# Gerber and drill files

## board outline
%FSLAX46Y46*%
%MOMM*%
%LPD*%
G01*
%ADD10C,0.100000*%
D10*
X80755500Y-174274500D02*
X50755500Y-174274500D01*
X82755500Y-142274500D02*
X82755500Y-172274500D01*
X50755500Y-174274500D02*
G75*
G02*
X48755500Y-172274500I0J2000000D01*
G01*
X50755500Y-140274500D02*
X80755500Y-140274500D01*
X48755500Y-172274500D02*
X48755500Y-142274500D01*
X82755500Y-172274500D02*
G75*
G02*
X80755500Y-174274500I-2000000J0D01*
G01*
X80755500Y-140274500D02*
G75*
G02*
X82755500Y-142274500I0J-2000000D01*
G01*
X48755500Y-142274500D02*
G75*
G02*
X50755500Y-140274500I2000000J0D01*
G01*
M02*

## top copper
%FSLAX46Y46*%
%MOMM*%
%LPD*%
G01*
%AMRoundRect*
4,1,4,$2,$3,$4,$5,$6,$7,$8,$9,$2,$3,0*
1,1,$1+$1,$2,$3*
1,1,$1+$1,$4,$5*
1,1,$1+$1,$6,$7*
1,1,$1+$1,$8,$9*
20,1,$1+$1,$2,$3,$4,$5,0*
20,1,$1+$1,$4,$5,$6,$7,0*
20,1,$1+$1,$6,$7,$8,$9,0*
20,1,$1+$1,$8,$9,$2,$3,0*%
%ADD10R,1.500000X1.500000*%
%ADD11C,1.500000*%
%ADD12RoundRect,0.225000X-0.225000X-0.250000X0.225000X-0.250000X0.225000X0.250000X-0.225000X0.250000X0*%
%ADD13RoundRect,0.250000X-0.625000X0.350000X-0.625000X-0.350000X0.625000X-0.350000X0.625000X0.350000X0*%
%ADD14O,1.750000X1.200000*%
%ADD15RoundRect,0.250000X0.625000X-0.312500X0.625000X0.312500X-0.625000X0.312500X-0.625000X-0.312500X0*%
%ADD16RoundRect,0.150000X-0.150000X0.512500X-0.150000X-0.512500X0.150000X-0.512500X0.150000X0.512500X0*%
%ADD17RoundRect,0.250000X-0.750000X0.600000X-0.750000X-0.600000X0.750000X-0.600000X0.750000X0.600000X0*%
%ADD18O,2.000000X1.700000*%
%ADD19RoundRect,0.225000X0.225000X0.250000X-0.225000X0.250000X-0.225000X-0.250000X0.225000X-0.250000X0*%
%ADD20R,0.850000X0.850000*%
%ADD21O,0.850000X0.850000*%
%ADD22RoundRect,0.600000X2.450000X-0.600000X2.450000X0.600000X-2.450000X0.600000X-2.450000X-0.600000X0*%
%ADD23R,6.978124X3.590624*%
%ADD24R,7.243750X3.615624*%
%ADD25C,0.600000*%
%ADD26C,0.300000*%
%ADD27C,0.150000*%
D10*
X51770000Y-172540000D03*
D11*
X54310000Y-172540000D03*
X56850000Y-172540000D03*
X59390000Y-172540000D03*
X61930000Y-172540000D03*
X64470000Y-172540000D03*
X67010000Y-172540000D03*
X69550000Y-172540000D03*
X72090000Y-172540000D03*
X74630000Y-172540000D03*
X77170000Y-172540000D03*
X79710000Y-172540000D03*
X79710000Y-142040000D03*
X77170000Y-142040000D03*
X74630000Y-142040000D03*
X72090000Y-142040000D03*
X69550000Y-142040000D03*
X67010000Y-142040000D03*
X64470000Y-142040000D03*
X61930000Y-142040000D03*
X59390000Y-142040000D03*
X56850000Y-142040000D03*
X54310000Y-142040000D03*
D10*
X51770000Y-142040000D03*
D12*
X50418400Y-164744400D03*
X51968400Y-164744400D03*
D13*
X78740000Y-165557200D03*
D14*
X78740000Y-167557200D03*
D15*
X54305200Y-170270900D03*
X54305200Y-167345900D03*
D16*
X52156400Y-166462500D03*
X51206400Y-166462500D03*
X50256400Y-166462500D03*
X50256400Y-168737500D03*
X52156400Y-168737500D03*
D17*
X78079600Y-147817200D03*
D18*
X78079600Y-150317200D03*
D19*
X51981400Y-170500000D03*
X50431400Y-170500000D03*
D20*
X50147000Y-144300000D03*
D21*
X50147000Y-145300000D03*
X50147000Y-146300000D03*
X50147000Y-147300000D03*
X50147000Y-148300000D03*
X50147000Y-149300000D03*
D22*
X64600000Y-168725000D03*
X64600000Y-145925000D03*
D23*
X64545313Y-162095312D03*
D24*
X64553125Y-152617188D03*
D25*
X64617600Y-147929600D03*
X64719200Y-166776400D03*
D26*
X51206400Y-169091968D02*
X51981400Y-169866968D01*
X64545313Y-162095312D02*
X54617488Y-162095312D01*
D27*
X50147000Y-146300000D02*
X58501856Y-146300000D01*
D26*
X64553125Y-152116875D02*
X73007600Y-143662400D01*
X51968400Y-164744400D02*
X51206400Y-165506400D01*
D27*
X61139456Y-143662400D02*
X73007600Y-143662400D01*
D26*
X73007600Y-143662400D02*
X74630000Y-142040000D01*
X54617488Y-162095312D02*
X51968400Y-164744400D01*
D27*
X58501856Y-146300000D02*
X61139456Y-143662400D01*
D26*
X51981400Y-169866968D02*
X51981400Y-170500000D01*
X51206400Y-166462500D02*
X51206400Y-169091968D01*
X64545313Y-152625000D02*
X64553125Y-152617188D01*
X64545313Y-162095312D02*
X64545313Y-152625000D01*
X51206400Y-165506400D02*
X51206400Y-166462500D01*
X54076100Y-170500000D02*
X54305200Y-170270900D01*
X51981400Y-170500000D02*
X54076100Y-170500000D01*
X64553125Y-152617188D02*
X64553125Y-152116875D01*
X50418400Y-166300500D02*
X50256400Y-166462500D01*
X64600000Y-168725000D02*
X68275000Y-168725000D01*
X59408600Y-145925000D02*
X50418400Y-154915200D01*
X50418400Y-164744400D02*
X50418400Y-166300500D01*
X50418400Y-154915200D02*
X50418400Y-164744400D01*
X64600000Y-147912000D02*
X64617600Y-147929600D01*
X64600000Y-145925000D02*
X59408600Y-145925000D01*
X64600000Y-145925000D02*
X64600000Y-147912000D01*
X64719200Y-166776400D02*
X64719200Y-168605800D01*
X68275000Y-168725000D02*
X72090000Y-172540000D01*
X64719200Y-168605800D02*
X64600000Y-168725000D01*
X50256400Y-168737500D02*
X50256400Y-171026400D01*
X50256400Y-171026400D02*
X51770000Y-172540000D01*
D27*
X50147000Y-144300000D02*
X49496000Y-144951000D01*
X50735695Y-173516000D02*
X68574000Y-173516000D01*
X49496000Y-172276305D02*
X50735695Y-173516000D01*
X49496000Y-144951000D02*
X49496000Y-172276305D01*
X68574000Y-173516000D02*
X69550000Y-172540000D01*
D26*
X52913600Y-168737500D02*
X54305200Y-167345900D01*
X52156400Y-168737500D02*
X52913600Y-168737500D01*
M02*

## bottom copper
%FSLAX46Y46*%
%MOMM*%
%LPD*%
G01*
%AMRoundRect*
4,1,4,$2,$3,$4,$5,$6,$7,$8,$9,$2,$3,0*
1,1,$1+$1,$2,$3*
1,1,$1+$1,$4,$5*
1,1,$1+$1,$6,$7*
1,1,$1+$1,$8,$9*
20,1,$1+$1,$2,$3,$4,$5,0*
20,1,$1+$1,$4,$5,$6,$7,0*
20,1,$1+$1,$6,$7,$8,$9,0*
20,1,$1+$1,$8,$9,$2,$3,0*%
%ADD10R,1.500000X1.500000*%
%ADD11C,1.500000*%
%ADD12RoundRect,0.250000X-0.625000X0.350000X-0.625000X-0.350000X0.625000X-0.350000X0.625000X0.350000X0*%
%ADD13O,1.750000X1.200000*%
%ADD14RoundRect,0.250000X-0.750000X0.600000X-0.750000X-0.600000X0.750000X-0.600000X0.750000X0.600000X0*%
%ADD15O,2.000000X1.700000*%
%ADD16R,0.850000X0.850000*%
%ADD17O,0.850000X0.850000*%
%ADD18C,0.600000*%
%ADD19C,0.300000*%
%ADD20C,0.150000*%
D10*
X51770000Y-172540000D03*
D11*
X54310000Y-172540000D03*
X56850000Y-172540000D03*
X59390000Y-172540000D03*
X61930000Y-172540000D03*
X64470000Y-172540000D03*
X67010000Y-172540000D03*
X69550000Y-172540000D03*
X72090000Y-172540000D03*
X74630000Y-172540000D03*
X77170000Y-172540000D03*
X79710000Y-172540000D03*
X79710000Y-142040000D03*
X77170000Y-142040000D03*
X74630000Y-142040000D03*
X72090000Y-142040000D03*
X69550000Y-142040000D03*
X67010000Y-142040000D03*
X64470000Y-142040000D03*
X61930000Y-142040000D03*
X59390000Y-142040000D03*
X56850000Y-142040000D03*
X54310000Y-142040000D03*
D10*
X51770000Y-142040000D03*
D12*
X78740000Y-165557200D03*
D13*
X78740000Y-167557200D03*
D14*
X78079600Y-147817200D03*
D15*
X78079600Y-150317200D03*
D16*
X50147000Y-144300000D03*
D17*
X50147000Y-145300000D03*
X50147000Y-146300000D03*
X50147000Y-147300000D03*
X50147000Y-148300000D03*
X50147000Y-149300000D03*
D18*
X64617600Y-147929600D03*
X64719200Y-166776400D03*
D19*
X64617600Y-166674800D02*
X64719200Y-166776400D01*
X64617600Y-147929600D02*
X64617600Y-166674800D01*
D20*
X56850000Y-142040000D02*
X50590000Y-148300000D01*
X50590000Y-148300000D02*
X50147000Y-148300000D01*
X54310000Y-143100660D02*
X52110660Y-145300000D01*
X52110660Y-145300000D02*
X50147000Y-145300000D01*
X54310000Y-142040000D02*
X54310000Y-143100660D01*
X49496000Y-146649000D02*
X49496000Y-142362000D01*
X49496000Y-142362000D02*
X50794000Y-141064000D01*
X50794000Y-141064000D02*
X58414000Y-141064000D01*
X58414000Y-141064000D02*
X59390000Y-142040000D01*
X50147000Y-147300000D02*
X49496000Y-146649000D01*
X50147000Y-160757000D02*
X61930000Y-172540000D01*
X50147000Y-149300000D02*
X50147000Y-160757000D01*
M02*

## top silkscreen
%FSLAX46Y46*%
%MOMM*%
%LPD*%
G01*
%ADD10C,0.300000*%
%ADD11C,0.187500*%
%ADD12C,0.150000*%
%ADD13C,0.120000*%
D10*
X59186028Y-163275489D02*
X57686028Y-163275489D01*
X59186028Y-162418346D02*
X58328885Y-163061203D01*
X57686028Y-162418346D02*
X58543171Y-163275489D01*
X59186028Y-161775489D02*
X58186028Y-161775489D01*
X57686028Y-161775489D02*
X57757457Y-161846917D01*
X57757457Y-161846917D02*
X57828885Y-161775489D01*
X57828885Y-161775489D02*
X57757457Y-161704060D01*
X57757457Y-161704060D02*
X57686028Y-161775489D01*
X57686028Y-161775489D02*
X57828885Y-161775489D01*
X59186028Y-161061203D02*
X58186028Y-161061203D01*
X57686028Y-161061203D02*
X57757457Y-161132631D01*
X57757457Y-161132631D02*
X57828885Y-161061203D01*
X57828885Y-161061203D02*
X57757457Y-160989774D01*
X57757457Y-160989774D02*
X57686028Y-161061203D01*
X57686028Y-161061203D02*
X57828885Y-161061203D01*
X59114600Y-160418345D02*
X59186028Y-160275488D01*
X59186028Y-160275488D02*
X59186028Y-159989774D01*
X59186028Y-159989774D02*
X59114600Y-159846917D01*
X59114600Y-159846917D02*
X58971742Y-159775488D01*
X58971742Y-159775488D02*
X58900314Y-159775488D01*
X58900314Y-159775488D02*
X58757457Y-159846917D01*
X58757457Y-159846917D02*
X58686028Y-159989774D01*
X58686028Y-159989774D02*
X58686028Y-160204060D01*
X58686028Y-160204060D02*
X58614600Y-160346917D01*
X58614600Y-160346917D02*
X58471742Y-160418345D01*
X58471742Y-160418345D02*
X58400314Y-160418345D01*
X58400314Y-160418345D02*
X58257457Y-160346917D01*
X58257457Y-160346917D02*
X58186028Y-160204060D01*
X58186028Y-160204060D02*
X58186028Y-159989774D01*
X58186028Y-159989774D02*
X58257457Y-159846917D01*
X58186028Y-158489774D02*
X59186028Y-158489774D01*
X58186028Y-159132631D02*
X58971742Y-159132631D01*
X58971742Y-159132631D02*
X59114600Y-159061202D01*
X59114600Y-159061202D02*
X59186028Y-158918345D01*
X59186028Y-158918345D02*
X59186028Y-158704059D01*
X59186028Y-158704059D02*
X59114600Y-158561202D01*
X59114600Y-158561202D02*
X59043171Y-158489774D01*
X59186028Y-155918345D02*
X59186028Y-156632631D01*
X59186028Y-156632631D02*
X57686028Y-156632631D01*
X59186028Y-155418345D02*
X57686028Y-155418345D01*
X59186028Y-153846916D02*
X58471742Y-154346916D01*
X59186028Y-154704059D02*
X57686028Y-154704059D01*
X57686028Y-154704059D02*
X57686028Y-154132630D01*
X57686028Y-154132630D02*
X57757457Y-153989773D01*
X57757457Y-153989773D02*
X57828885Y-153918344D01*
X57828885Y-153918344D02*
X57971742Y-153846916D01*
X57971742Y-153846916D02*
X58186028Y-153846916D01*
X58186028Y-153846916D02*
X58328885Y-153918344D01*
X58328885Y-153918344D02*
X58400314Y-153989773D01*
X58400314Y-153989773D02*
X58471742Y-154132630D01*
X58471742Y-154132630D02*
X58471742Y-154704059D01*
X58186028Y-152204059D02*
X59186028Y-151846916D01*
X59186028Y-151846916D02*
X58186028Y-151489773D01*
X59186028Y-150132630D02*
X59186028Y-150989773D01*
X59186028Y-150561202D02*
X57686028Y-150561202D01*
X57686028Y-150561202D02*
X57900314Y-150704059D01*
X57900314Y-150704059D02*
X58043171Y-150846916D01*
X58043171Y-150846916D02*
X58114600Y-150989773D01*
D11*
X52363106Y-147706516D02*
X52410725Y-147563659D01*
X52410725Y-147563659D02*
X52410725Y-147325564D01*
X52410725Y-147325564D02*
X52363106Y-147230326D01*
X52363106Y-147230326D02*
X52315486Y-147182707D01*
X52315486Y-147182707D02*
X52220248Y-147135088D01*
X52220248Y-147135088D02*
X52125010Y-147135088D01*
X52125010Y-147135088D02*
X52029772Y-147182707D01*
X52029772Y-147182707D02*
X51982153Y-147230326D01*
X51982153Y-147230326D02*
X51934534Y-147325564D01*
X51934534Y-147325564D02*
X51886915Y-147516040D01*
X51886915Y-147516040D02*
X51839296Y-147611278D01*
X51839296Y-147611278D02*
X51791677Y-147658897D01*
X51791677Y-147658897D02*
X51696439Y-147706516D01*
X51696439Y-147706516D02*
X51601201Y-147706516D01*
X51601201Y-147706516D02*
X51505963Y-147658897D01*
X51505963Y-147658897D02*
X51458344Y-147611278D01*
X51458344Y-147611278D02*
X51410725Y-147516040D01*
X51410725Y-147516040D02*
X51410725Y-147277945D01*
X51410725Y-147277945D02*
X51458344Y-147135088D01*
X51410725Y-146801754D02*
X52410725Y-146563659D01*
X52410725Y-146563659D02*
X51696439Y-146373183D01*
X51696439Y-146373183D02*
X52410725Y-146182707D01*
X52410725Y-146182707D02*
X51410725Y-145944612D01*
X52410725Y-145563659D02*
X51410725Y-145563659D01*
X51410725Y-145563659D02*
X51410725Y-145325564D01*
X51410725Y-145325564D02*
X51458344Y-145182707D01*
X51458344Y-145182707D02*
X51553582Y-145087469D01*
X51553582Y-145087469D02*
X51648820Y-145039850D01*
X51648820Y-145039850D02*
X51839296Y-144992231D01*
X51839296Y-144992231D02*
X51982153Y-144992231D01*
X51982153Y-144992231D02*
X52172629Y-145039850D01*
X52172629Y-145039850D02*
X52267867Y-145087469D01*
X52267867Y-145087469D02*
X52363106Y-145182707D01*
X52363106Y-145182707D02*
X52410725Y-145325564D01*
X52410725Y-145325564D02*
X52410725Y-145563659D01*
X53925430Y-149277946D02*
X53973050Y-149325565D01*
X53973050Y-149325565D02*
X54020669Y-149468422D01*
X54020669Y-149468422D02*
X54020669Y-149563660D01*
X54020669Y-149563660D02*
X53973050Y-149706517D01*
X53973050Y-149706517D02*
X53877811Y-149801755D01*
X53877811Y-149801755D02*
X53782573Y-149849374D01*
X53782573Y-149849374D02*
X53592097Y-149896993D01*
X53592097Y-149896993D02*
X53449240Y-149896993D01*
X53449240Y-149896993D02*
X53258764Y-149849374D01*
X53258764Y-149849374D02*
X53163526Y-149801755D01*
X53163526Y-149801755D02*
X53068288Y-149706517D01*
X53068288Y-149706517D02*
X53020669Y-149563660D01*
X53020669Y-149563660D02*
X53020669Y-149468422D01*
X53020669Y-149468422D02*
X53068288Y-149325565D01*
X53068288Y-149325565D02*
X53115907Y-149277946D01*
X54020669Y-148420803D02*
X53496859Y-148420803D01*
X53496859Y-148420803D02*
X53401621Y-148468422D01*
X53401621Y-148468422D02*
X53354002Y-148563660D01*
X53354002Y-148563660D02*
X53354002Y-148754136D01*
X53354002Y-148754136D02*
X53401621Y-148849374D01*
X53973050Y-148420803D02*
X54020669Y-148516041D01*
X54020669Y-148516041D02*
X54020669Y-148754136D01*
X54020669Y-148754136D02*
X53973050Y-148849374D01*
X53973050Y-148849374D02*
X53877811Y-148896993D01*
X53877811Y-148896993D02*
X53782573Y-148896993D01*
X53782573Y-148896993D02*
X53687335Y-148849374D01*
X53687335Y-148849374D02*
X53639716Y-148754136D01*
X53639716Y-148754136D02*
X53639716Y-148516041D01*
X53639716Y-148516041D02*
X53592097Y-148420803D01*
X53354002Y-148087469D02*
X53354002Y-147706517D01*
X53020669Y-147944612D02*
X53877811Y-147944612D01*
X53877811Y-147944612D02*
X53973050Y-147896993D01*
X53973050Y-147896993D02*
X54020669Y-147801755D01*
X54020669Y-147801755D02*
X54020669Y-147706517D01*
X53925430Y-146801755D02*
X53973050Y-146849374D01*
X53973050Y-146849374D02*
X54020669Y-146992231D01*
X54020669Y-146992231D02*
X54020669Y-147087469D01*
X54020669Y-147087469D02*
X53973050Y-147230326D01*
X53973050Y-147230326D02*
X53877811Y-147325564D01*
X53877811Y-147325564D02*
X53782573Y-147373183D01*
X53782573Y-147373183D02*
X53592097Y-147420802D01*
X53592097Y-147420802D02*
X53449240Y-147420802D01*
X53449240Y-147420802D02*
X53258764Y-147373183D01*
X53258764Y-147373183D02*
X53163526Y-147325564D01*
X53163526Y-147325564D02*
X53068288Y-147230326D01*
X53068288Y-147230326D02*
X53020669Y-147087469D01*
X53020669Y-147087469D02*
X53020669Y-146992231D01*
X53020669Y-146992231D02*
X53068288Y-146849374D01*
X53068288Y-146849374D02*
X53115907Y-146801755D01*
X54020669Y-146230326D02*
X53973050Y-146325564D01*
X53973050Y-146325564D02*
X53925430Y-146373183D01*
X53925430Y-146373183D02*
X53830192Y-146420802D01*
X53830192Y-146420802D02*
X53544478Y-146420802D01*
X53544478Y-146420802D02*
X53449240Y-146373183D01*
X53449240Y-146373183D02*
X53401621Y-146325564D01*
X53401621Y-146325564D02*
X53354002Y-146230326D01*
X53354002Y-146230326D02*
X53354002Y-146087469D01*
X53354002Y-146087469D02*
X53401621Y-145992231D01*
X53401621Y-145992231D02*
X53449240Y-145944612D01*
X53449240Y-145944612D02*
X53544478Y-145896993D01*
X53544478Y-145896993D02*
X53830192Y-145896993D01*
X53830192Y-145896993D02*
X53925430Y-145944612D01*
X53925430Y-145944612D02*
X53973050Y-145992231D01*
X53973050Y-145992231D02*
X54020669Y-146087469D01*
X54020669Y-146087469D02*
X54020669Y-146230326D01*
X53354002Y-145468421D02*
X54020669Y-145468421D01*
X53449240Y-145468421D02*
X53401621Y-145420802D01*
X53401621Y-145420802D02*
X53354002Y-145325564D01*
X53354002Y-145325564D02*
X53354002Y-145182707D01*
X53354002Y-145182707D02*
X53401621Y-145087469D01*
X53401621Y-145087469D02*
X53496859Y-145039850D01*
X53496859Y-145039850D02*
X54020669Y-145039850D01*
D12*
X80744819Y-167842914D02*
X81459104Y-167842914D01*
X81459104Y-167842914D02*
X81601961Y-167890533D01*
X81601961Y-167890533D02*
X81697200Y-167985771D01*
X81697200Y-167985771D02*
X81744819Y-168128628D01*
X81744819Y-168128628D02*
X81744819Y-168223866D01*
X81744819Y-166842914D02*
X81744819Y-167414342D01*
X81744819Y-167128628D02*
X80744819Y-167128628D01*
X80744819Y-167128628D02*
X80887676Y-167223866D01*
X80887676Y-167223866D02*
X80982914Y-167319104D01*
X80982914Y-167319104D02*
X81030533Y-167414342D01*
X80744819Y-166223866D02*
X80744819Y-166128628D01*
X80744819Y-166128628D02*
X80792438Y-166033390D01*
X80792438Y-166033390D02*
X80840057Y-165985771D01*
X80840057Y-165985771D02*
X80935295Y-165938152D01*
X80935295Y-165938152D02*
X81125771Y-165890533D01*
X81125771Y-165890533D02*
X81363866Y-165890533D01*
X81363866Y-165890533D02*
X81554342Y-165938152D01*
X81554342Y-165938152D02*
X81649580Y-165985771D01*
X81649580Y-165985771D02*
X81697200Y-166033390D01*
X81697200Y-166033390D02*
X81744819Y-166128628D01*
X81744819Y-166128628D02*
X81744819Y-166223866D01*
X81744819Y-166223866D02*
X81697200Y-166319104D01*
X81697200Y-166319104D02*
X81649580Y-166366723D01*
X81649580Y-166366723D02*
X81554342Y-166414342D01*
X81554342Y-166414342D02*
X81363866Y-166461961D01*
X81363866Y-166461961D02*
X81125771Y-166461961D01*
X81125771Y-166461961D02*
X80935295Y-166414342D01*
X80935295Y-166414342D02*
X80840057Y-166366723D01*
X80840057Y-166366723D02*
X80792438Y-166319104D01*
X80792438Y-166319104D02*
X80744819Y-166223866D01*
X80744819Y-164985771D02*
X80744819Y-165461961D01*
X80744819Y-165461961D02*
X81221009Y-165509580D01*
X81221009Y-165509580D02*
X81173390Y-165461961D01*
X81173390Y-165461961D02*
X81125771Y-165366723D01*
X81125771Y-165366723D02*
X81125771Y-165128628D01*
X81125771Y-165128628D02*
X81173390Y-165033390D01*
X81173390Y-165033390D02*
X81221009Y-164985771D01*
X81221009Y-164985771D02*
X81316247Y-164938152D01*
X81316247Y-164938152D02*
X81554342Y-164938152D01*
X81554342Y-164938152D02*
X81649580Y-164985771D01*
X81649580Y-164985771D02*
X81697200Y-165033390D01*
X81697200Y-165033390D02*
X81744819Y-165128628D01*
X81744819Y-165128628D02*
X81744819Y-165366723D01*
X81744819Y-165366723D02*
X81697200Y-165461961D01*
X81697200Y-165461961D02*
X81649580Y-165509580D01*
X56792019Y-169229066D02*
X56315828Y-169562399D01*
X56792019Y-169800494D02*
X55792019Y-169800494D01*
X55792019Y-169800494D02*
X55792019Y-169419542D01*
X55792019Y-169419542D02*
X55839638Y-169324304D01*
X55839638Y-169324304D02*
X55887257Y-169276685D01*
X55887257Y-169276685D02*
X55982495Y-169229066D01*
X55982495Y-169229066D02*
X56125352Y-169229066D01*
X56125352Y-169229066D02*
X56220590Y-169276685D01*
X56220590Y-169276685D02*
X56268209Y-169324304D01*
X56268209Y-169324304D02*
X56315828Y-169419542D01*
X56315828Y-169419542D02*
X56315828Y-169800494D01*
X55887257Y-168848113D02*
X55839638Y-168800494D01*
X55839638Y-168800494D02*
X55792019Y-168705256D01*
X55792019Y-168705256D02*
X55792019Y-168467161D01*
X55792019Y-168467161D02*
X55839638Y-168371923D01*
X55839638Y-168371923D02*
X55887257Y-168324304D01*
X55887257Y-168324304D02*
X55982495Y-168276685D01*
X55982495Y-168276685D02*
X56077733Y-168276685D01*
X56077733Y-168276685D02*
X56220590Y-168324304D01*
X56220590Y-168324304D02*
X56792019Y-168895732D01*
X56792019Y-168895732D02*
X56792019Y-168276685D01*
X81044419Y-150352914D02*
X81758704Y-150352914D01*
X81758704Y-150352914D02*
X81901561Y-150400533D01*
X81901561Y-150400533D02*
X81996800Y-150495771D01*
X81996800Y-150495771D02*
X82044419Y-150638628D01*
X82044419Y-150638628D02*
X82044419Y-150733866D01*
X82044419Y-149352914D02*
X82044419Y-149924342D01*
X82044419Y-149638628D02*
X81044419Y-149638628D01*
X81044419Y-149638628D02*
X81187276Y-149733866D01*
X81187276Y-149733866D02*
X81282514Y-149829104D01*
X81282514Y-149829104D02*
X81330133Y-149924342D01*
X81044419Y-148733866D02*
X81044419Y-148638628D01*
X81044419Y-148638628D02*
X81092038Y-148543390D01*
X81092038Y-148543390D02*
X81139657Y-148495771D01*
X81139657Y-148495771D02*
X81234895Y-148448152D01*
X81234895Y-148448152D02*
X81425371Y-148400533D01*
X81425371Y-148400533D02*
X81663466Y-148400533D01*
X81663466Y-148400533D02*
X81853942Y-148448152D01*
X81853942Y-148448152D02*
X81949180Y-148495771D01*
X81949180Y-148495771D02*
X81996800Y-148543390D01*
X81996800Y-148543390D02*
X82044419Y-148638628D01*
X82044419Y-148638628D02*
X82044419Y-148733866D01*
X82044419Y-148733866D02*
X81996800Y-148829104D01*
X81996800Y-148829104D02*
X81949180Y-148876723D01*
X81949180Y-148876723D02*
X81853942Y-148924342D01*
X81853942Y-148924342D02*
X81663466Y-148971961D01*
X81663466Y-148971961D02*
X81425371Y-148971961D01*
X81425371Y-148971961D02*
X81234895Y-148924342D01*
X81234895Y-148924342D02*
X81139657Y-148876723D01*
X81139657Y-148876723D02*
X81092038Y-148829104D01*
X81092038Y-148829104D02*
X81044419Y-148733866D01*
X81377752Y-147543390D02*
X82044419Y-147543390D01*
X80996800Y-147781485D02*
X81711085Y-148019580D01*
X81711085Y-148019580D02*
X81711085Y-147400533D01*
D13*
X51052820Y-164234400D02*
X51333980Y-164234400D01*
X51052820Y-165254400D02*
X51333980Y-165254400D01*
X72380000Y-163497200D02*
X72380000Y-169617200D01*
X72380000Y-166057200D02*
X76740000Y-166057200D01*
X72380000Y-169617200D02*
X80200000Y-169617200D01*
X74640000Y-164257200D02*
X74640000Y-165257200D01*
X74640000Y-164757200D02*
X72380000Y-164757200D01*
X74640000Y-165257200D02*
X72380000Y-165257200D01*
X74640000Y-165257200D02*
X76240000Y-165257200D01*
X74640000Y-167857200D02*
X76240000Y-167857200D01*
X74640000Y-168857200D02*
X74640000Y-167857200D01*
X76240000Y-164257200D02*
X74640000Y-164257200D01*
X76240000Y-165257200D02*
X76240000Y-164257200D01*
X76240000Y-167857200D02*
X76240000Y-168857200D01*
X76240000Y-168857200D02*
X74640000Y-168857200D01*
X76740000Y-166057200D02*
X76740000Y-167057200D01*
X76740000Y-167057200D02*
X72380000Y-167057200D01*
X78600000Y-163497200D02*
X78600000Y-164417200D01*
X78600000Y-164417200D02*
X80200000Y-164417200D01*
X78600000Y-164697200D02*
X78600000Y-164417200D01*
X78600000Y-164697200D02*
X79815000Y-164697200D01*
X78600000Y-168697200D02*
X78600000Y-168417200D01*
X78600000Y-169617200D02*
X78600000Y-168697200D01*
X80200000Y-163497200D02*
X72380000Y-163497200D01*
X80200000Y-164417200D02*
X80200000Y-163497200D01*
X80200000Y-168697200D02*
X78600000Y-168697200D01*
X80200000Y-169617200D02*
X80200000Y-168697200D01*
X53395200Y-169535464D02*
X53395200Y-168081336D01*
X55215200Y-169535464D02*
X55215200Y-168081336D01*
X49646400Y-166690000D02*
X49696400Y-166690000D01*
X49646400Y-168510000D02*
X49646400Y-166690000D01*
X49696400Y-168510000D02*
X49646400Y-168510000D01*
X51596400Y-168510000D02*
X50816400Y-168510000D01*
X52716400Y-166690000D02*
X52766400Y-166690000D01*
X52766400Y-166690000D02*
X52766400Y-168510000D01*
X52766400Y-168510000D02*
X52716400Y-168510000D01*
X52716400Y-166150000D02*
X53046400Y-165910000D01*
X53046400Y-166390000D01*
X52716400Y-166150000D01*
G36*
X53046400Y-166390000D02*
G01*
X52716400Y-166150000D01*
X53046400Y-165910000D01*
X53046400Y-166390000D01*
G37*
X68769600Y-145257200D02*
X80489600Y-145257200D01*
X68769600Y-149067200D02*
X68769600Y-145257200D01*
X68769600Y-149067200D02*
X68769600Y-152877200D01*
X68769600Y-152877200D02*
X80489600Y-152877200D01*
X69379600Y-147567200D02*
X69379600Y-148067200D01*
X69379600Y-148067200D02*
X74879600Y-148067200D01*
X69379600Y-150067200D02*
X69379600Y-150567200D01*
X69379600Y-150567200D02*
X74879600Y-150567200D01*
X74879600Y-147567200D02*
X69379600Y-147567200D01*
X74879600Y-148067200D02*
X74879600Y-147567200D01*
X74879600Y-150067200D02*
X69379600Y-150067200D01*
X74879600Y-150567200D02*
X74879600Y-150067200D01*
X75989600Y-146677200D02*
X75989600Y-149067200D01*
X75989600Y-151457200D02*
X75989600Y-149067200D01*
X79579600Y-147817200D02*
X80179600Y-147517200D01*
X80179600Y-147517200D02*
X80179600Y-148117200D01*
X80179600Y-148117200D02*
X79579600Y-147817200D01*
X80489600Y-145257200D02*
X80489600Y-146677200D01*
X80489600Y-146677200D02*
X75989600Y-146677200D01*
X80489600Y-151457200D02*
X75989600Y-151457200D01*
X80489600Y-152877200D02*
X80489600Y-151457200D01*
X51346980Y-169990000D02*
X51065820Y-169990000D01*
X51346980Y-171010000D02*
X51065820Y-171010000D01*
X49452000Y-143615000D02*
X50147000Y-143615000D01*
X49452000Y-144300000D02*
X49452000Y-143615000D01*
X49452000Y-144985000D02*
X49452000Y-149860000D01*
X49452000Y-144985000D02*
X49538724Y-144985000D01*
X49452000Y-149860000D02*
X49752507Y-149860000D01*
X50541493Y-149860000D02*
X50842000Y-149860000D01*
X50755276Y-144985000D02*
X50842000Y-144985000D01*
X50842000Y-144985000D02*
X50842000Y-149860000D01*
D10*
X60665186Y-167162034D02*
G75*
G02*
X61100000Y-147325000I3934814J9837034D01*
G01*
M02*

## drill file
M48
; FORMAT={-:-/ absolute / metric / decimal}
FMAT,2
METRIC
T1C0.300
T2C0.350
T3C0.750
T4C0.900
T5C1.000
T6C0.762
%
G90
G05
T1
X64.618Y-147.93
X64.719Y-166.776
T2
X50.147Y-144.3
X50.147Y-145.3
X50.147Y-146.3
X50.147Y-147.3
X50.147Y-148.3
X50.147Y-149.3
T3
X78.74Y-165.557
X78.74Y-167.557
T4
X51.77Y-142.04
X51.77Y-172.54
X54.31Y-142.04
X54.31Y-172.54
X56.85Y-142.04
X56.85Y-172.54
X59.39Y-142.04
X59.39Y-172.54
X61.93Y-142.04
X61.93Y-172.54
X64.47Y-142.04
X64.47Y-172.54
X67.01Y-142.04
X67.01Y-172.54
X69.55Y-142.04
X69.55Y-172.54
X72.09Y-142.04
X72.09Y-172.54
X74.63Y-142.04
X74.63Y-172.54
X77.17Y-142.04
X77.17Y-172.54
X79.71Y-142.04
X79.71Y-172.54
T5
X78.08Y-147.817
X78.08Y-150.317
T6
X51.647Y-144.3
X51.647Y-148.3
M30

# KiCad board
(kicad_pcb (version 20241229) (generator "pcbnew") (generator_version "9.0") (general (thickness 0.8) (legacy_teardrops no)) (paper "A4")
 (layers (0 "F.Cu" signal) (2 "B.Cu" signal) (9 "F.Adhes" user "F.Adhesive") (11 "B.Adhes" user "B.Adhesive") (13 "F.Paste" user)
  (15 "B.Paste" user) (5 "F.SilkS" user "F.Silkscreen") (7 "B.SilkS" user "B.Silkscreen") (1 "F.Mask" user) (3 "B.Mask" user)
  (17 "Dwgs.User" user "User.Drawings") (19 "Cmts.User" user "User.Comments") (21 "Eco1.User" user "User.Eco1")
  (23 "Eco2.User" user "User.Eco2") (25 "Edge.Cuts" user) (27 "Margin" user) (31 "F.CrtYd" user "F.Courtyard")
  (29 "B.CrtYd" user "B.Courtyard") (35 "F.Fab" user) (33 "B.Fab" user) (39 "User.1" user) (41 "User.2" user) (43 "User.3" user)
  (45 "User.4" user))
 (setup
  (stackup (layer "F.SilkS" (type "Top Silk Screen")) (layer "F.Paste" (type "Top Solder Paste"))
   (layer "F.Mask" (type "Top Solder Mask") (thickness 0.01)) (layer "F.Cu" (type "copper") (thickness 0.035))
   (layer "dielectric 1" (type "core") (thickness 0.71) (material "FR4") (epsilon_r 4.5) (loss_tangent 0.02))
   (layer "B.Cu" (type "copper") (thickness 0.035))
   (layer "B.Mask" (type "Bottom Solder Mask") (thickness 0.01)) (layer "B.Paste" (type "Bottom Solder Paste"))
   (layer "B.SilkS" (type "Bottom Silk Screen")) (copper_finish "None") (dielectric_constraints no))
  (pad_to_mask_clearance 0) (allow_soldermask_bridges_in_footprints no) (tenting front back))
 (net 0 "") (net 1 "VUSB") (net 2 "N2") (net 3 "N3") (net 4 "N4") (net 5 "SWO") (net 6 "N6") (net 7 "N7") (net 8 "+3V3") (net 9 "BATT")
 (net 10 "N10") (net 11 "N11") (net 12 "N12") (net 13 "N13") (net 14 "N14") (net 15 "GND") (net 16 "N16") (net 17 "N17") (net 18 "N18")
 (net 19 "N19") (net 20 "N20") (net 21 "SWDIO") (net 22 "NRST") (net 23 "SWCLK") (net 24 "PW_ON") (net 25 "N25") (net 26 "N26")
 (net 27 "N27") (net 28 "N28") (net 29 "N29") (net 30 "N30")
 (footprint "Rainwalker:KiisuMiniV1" (layer "F.Cu") (at 65.74 157.29)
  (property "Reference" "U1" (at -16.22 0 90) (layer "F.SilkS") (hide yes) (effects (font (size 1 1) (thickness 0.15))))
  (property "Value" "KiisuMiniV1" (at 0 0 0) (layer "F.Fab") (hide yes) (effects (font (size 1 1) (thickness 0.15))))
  (pad "1" thru_hole rect (at -13.97 15.25) (size 1.5 1.5) (drill 0.9) (layers "*.Cu" "*.Mask") (remove_unused_layers no) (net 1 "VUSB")
   (thermal_bridge_angle 45))
  (pad "2" thru_hole circle (at -11.43 15.25) (size 1.5 1.5) (drill 0.9) (layers "*.Cu" "*.Mask") (remove_unused_layers no) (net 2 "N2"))
  (pad "3" thru_hole circle (at -8.89 15.25) (size 1.5 1.5) (drill 0.9) (layers "*.Cu" "*.Mask") (remove_unused_layers no) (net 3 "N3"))
  (pad "4" thru_hole circle (at -6.35 15.25) (size 1.5 1.5) (drill 0.9) (layers "*.Cu" "*.Mask") (remove_unused_layers no) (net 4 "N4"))
  (pad "5" thru_hole circle (at -3.81 15.25) (size 1.5 1.5) (drill 0.9) (layers "*.Cu" "*.Mask") (remove_unused_layers no) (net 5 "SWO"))
  (pad "6" thru_hole circle (at -1.27 15.25) (size 1.5 1.5) (drill 0.9) (layers "*.Cu" "*.Mask") (remove_unused_layers no) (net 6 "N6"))
  (pad "7" thru_hole circle (at 1.27 15.25) (size 1.5 1.5) (drill 0.9) (layers "*.Cu" "*.Mask") (remove_unused_layers no) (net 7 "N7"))
  (pad "8" thru_hole circle (at 3.81 15.25) (size 1.5 1.5) (drill 0.9) (layers "*.Cu" "*.Mask") (remove_unused_layers no) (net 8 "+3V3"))
  (pad "9" thru_hole circle (at 6.35 15.25) (size 1.5 1.5) (drill 0.9) (layers "*.Cu" "*.Mask") (remove_unused_layers no) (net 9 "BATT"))
  (pad "10" thru_hole circle (at 8.89 15.25) (size 1.5 1.5) (drill 0.9) (layers "*.Cu" "*.Mask") (remove_unused_layers no) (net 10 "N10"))
  (pad "11" thru_hole circle (at 11.43 15.25) (size 1.5 1.5) (drill 0.9) (layers "*.Cu" "*.Mask") (remove_unused_layers no) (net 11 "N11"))
  (pad "12" thru_hole circle (at 13.97 15.25) (size 1.5 1.5) (drill 0.9) (layers "*.Cu" "*.Mask") (remove_unused_layers no) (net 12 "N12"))
  (pad "13" thru_hole circle (at 13.97 -15.25) (size 1.5 1.5) (drill 0.9) (layers "*.Cu" "*.Mask") (remove_unused_layers no) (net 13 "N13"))
  (pad "14" thru_hole circle (at 11.43 -15.25) (size 1.5 1.5) (drill 0.9) (layers "*.Cu" "*.Mask") (remove_unused_layers no) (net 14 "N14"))
  (pad "15" thru_hole circle (at 8.89 -15.25) (size 1.5 1.5) (drill 0.9) (layers "*.Cu" "*.Mask") (remove_unused_layers no) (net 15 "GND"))
  (pad "16" thru_hole circle (at 6.35 -15.25) (size 1.5 1.5) (drill 0.9) (layers "*.Cu" "*.Mask") (remove_unused_layers no) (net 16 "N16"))
  (pad "17" thru_hole circle (at 3.81 -15.25) (size 1.5 1.5) (drill 0.9) (layers "*.Cu" "*.Mask") (remove_unused_layers no) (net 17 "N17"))
  (pad "18" thru_hole circle (at 1.27 -15.25) (size 1.5 1.5) (drill 0.9) (layers "*.Cu" "*.Mask") (remove_unused_layers no) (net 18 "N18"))
  (pad "19" thru_hole circle (at -1.27 -15.25) (size 1.5 1.5) (drill 0.9) (layers "*.Cu" "*.Mask") (remove_unused_layers no) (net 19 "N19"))
  (pad "20" thru_hole circle (at -3.81 -15.25) (size 1.5 1.5) (drill 0.9) (layers "*.Cu" "*.Mask") (remove_unused_layers no) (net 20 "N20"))
  (pad "21" thru_hole circle (at -6.35 -15.25) (size 1.5 1.5) (drill 0.9) (layers "*.Cu" "*.Mask") (remove_unused_layers no)
   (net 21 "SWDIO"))
  (pad "22" thru_hole circle (at -8.89 -15.25) (size 1.5 1.5) (drill 0.9) (layers "*.Cu" "*.Mask") (remove_unused_layers no) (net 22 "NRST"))
  (pad "23" thru_hole circle (at -11.43 -15.25) (size 1.5 1.5) (drill 0.9) (layers "*.Cu" "*.Mask") (remove_unused_layers no)
   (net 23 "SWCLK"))
  (pad "24" thru_hole rect (at -13.97 -15.25) (size 1.5 1.5) (drill 0.9) (layers "*.Cu" "*.Mask") (remove_unused_layers no) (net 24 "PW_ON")
   (thermal_bridge_angle 45)))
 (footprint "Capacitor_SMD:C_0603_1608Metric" (layer "F.Cu") (at 51.1934 164.7444)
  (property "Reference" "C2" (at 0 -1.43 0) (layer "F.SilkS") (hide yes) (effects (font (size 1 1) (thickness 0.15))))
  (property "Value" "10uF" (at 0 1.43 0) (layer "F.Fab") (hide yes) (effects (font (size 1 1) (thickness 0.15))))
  (fp_line (start -0.14058 -0.51) (end 0.14058 -0.51) (stroke (width 0.12) (type solid)) (layer "F.SilkS"))
  (fp_line (start -0.14058 0.51) (end 0.14058 0.51) (stroke (width 0.12) (type solid)) (layer "F.SilkS"))
  (pad "1" smd roundrect (at -0.775 0) (size 0.9 0.95) (layers "F.Cu" "F.Mask" "F.Paste") (roundrect_rratio 0.25) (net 9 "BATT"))
  (pad "2" smd roundrect (at 0.775 0) (size 0.9 0.95) (layers "F.Cu" "F.Mask" "F.Paste") (roundrect_rratio 0.25) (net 15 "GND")))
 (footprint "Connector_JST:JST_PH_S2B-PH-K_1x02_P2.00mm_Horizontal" (layer "F.Cu") (at 78.74 165.5572 -90)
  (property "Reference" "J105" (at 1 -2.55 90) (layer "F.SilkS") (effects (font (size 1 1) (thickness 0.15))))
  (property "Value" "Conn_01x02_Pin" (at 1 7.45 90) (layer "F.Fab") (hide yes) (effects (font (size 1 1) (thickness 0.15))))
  (fp_line (start -2.06 6.36) (end 4.06 6.36) (stroke (width 0.12) (type solid)) (layer "F.SilkS"))
  (fp_line (start 0.5 6.36) (end 0.5 2) (stroke (width 0.12) (type solid)) (layer "F.SilkS"))
  (fp_line (start 4.06 6.36) (end 4.06 -1.46) (stroke (width 0.12) (type solid)) (layer "F.SilkS"))
  (fp_line (start -1.3 4.1) (end -0.3 4.1) (stroke (width 0.12) (type solid)) (layer "F.SilkS"))
  (fp_line (start -0.8 4.1) (end -0.8 6.36) (stroke (width 0.12) (type solid)) (layer "F.SilkS"))
  (fp_line (start -0.3 4.1) (end -0.3 6.36) (stroke (width 0.12) (type solid)) (layer "F.SilkS"))
  (fp_line (start -0.3 4.1) (end -0.3 2.5) (stroke (width 0.12) (type solid)) (layer "F.SilkS"))
  (fp_line (start 2.3 4.1) (end 2.3 2.5) (stroke (width 0.12) (type solid)) (layer "F.SilkS"))
  (fp_line (start 3.3 4.1) (end 2.3 4.1) (stroke (width 0.12) (type solid)) (layer "F.SilkS"))
  (fp_line (start -1.3 2.5) (end -1.3 4.1) (stroke (width 0.12) (type solid)) (layer "F.SilkS"))
  (fp_line (start -0.3 2.5) (end -1.3 2.5) (stroke (width 0.12) (type solid)) (layer "F.SilkS"))
  (fp_line (start 2.3 2.5) (end 3.3 2.5) (stroke (width 0.12) (type solid)) (layer "F.SilkS"))
  (fp_line (start 3.3 2.5) (end 3.3 4.1) (stroke (width 0.12) (type solid)) (layer "F.SilkS"))
  (fp_line (start 0.5 2) (end 1.5 2) (stroke (width 0.12) (type solid)) (layer "F.SilkS"))
  (fp_line (start 1.5 2) (end 1.5 6.36) (stroke (width 0.12) (type solid)) (layer "F.SilkS"))
  (fp_line (start -2.06 0.14) (end -1.14 0.14) (stroke (width 0.12) (type solid)) (layer "F.SilkS"))
  (fp_line (start -1.14 0.14) (end -1.14 -1.46) (stroke (width 0.12) (type solid)) (layer "F.SilkS"))
  (fp_line (start -0.86 0.14) (end -1.14 0.14) (stroke (width 0.12) (type solid)) (layer "F.SilkS"))
  (fp_line (start -0.86 0.14) (end -0.86 -1.075) (stroke (width 0.12) (type solid)) (layer "F.SilkS"))
  (fp_line (start 3.14 0.14) (end 2.86 0.14) (stroke (width 0.12) (type solid)) (layer "F.SilkS"))
  (fp_line (start 4.06 0.14) (end 3.14 0.14) (stroke (width 0.12) (type solid)) (layer "F.SilkS"))
  (fp_line (start -2.06 -1.46) (end -2.06 6.36) (stroke (width 0.12) (type solid)) (layer "F.SilkS"))
  (fp_line (start -1.14 -1.46) (end -2.06 -1.46) (stroke (width 0.12) (type solid)) (layer "F.SilkS"))
  (fp_line (start 3.14 -1.46) (end 3.14 0.14) (stroke (width 0.12) (type solid)) (layer "F.SilkS"))
  (fp_line (start 4.06 -1.46) (end 3.14 -1.46) (stroke (width 0.12) (type solid)) (layer "F.SilkS"))
  (pad "1" thru_hole roundrect (at 0 0 270) (size 1.2 1.75) (drill 0.75) (layers "*.Cu" "*.Mask") (remove_unused_layers no)
   (roundrect_rratio 0.208333) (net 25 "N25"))
  (pad "2" thru_hole oval (at 2 0 270) (size 1.2 1.75) (drill 0.75) (layers "*.Cu" "*.Mask") (remove_unused_layers no) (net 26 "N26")))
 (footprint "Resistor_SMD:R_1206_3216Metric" (layer "F.Cu") (at 54.3052 168.8084 90)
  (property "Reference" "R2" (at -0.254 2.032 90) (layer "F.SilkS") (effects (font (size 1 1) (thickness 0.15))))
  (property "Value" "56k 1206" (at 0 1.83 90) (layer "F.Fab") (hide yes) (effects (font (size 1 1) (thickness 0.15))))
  (fp_line (start -0.727064 -0.91) (end 0.727064 -0.91) (stroke (width 0.12) (type solid)) (layer "F.SilkS"))
  (fp_line (start -0.727064 0.91) (end 0.727064 0.91) (stroke (width 0.12) (type solid)) (layer "F.SilkS"))
  (pad "1" smd roundrect (at -1.4625 0 90) (size 1.125 1.75) (layers "F.Cu" "F.Mask" "F.Paste") (roundrect_rratio 0.222222) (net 15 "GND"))
  (pad "2" smd roundrect (at 1.4625 0 90) (size 1.125 1.75) (layers "F.Cu" "F.Mask" "F.Paste") (roundrect_rratio 0.222222) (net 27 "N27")))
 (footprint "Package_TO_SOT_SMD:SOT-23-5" (layer "F.Cu") (at 51.2064 167.6 -90)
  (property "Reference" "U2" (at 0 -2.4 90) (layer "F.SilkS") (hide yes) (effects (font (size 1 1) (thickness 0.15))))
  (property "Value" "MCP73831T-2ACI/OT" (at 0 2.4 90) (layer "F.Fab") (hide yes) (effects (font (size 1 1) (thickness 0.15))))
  (fp_line (start -0.91 1.56) (end -0.91 1.51) (stroke (width 0.12) (type solid)) (layer "F.SilkS"))
  (fp_line (start 0.91 1.56) (end -0.91 1.56) (stroke (width 0.12) (type solid)) (layer "F.SilkS"))
  (fp_line (start 0.91 1.51) (end 0.91 1.56) (stroke (width 0.12) (type solid)) (layer "F.SilkS"))
  (fp_line (start 0.91 -0.39) (end 0.91 0.39) (stroke (width 0.12) (type solid)) (layer "F.SilkS"))
  (fp_line (start -0.91 -1.51) (end -0.91 -1.56) (stroke (width 0.12) (type solid)) (layer "F.SilkS"))
  (fp_line (start -0.91 -1.56) (end 0.91 -1.56) (stroke (width 0.12) (type solid)) (layer "F.SilkS"))
  (fp_line (start 0.91 -1.56) (end 0.91 -1.51) (stroke (width 0.12) (type solid)) (layer "F.SilkS"))
  (fp_poly (pts (xy -1.45 -1.51) (xy -1.69 -1.84) (xy -1.21 -1.84)) (stroke (width 0.12) (type solid)) (fill yes) (layer "F.SilkS"))
  (pad "1" smd roundrect (at -1.1375 -0.95 270) (size 1.325 0.6) (layers "F.Cu" "F.Mask" "F.Paste") (roundrect_rratio 0.25) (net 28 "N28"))
  (pad "2" smd roundrect (at -1.1375 0 270) (size 1.325 0.6) (layers "F.Cu" "F.Mask" "F.Paste") (roundrect_rratio 0.25) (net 15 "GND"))
  (pad "3" smd roundrect (at -1.1375 0.95 270) (size 1.325 0.6) (layers "F.Cu" "F.Mask" "F.Paste") (roundrect_rratio 0.25) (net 9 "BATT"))
  (pad "4" smd roundrect (at 1.1375 0.95 270) (size 1.325 0.6) (layers "F.Cu" "F.Mask" "F.Paste") (roundrect_rratio 0.25) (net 1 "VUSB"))
  (pad "5" smd roundrect (at 1.1375 -0.95 270) (size 1.325 0.6) (layers "F.Cu" "F.Mask" "F.Paste") (roundrect_rratio 0.25) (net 27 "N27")))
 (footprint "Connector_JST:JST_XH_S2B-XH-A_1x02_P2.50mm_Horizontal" (layer "F.Cu") (at 78.0796 147.8172 -90)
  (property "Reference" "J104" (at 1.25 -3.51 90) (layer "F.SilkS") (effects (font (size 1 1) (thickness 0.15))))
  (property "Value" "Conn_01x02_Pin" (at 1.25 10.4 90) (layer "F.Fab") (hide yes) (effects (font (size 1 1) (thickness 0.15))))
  (fp_line (start -2.56 9.31) (end -2.56 -2.41) (stroke (width 0.12) (type solid)) (layer "F.SilkS"))
  (fp_line (start 1.25 9.31) (end -2.56 9.31) (stroke (width 0.12) (type solid)) (layer "F.SilkS"))
  (fp_line (start 1.25 9.31) (end 5.06 9.31) (stroke (width 0.12) (type solid)) (layer "F.SilkS"))
  (fp_line (start 5.06 9.31) (end 5.06 -2.41) (stroke (width 0.12) (type solid)) (layer "F.SilkS"))
  (fp_line (start -0.25 8.7) (end 0.25 8.7) (stroke (width 0.12) (type solid)) (layer "F.SilkS"))
  (fp_line (start 0.25 8.7) (end 0.25 3.2) (stroke (width 0.12) (type solid)) (layer "F.SilkS"))
  (fp_line (start 2.25 8.7) (end 2.75 8.7) (stroke (width 0.12) (type solid)) (layer "F.SilkS"))
  (fp_line (start 2.75 8.7) (end 2.75 3.2) (stroke (width 0.12) (type solid)) (layer "F.SilkS"))
  (fp_line (start -0.25 3.2) (end -0.25 8.7) (stroke (width 0.12) (type solid)) (layer "F.SilkS"))
  (fp_line (start 0.25 3.2) (end -0.25 3.2) (stroke (width 0.12) (type solid)) (layer "F.SilkS"))
  (fp_line (start 2.25 3.2) (end 2.25 8.7) (stroke (width 0.12) (type solid)) (layer "F.SilkS"))
  (fp_line (start 2.75 3.2) (end 2.25 3.2) (stroke (width 0.12) (type solid)) (layer "F.SilkS"))
  (fp_line (start -1.14 2.09) (end 1.25 2.09) (stroke (width 0.12) (type solid)) (layer "F.SilkS"))
  (fp_line (start 3.64 2.09) (end 1.25 2.09) (stroke (width 0.12) (type solid)) (layer "F.SilkS"))
  (fp_line (start 0 -1.5) (end -0.3 -2.1) (stroke (width 0.12) (type solid)) (layer "F.SilkS"))
  (fp_line (start -0.3 -2.1) (end 0.3 -2.1) (stroke (width 0.12) (type solid)) (layer "F.SilkS"))
  (fp_line (start 0.3 -2.1) (end 0 -1.5) (stroke (width 0.12) (type solid)) (layer "F.SilkS"))
  (fp_line (start -2.56 -2.41) (end -1.14 -2.41) (stroke (width 0.12) (type solid)) (layer "F.SilkS"))
  (fp_line (start -1.14 -2.41) (end -1.14 2.09) (stroke (width 0.12) (type solid)) (layer "F.SilkS"))
  (fp_line (start 3.64 -2.41) (end 3.64 2.09) (stroke (width 0.12) (type solid)) (layer "F.SilkS"))
  (fp_line (start 5.06 -2.41) (end 3.64 -2.41) (stroke (width 0.12) (type solid)) (layer "F.SilkS"))
  (pad "1" thru_hole roundrect (at 0 0 270) (size 1.7 2) (drill 1) (layers "*.Cu" "*.Mask") (remove_unused_layers no)
   (roundrect_rratio 0.147059) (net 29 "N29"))
  (pad "2" thru_hole oval (at 2.5 0 270) (size 1.7 2) (drill 1) (layers "*.Cu" "*.Mask") (remove_unused_layers no) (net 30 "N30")))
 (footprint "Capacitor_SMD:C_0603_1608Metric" (layer "F.Cu") (at 51.2064 170.5 180)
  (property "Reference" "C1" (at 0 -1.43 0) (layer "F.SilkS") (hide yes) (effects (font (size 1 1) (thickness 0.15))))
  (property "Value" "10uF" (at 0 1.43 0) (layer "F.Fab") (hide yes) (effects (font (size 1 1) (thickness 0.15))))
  (fp_line (start -0.14058 0.51) (end 0.14058 0.51) (stroke (width 0.12) (type solid)) (layer "F.SilkS"))
  (fp_line (start -0.14058 -0.51) (end 0.14058 -0.51) (stroke (width 0.12) (type solid)) (layer "F.SilkS"))
  (pad "1" smd roundrect (at -0.775 0 180) (size 0.9 0.95) (layers "F.Cu" "F.Mask" "F.Paste") (roundrect_rratio 0.25) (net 15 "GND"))
  (pad "2" smd roundrect (at 0.775 0 180) (size 0.9 0.95) (layers "F.Cu" "F.Mask" "F.Paste") (roundrect_rratio 0.25) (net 1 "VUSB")))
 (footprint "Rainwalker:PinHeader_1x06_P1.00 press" (layer "F.Cu") (at 50.147 144.3)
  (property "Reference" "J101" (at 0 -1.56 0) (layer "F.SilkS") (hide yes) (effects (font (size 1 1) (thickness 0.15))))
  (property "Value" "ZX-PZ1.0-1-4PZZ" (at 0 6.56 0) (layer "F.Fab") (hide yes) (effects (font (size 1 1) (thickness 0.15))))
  (fp_line (start -0.695 -0.685) (end 0 -0.685) (stroke (width 0.12) (type solid)) (layer "F.SilkS"))
  (fp_line (start -0.695 0) (end -0.695 -0.685) (stroke (width 0.12) (type solid)) (layer "F.SilkS"))
  (fp_line (start -0.695 0.685) (end -0.695 5.56) (stroke (width 0.12) (type solid)) (layer "F.SilkS"))
  (fp_line (start -0.695 0.685) (end -0.608276 0.685) (stroke (width 0.12) (type solid)) (layer "F.SilkS"))
  (fp_line (start -0.695 5.56) (end -0.394493 5.56) (stroke (width 0.12) (type solid)) (layer "F.SilkS"))
  (fp_line (start 0.394493 5.56) (end 0.695 5.56) (stroke (width 0.12) (type solid)) (layer "F.SilkS"))
  (fp_line (start 0.608276 0.685) (end 0.695 0.685) (stroke (width 0.12) (type solid)) (layer "F.SilkS"))
  (fp_line (start 0.695 0.685) (end 0.695 5.56) (stroke (width 0.12) (type solid)) (layer "F.SilkS"))
  (pad "" np_thru_hole circle (at 1.5 0) (size 0.5 0.5) (drill 0.762) (layers "*.Cu" "*.Mask"))
  (pad "" np_thru_hole circle (at 1.5 4) (size 0.5 0.5) (drill 0.762) (layers "*.Cu" "*.Mask"))
  (pad "1" thru_hole rect (at 0 0) (size 0.85 0.85) (drill 0.35) (layers "*.Cu" "*.Mask") (remove_unused_layers no) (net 8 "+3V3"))
  (pad "2" thru_hole oval (at 0 1) (size 0.85 0.85) (drill 0.35) (layers "*.Cu" "*.Mask") (remove_unused_layers no) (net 23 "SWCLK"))
  (pad "3" thru_hole oval (at 0 2) (size 0.85 0.85) (drill 0.35) (layers "*.Cu" "*.Mask") (remove_unused_layers no) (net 15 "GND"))
  (pad "4" thru_hole oval (at 0 3) (size 0.85 0.85) (drill 0.35) (layers "*.Cu" "*.Mask") (remove_unused_layers no) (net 21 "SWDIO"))
  (pad "5" thru_hole oval (at 0 4) (size 0.85 0.85) (drill 0.35) (layers "*.Cu" "*.Mask") (remove_unused_layers no) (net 22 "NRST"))
  (pad "6" thru_hole oval (at 0 5) (size 0.85 0.85) (drill 0.35) (layers "*.Cu" "*.Mask") (remove_unused_layers no) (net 5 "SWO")))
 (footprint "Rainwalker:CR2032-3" (layer "F.Cu") (at 64.6 157.325 90)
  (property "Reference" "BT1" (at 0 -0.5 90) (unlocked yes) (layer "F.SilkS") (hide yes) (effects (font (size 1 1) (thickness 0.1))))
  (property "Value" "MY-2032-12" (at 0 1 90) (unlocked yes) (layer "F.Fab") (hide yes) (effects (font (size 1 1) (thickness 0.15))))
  (fp_arc (start -9.837034 -3.934814) (mid 0.232175 -10.592266) (end 10 -3.5) (stroke (width 0.3) (type default)) (layer "F.SilkS"))
  (pad "+" smd roundrect (at -11.4 0 90) (size 2.4 6.1) (layers "F.Cu" "F.Mask" "F.Paste") (roundrect_rratio 0.25) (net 9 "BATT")
   (thermal_bridge_angle 45))
  (pad "+" smd roundrect (at 11.4 0 90) (size 2.4 6.1) (layers "F.Cu" "F.Mask" "F.Paste") (roundrect_rratio 0.25) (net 9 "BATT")
   (thermal_bridge_angle 45))
  (pad "-" smd rect (at -4.770312 -0.054687 90) (size 3.590624 6.978124) (layers "F.Cu" "F.Mask") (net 15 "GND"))
  (pad "-" smd rect (at 4.707812 -0.046875 90) (size 3.615624 7.24375) (layers "F.Cu" "F.Mask") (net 15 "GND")))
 (gr_line (start 80.7555 174.2745) (end 50.7555 174.2745) (stroke (width 0.1) (type default)) (layer "Edge.Cuts"))
 (gr_line (start 82.7555 142.2745) (end 82.7555 172.2745) (stroke (width 0.1) (type default)) (layer "Edge.Cuts"))
 (gr_arc (start 50.7555 174.2745) (mid 49.341286 173.688714) (end 48.7555 172.2745) (stroke (width 0.1) (type default)) (layer "Edge.Cuts"))
 (gr_line (start 50.7555 140.2745) (end 80.7555 140.2745) (stroke (width 0.1) (type default)) (layer "Edge.Cuts"))
 (gr_line (start 48.7555 172.2745) (end 48.7555 142.2745) (stroke (width 0.1) (type default)) (layer "Edge.Cuts"))
 (gr_arc (start 82.7555 172.2745) (mid 82.169714 173.688714) (end 80.7555 174.2745) (stroke (width 0.1) (type default)) (layer "Edge.Cuts"))
 (gr_arc (start 80.7555 140.2745) (mid 82.169714 140.860286) (end 82.7555 142.2745) (stroke (width 0.1) (type default)) (layer "Edge.Cuts"))
 (gr_arc (start 48.7555 142.2745) (mid 49.341286 140.860286) (end 50.7555 140.2745) (stroke (width 0.1) (type default)) (layer "Edge.Cuts"))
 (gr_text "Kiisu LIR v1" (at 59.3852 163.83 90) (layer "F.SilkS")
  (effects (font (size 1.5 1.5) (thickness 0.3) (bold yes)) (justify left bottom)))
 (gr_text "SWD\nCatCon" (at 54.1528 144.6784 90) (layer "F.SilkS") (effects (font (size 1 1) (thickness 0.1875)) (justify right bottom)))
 (segment (start 51.2064 169.091968) (end 51.9814 169.866968) (width 0.3) (layer "F.Cu") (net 15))
 (segment (start 64.545313 162.095312) (end 54.617488 162.095312) (width 0.3) (layer "F.Cu") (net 15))
 (segment (start 50.147 146.3) (end 58.501856 146.3) (width 0.15) (layer "F.Cu") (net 15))
 (segment (start 64.553125 152.116875) (end 73.0076 143.6624) (width 0.3) (layer "F.Cu") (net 15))
 (segment (start 51.9684 164.7444) (end 51.2064 165.5064) (width 0.3) (layer "F.Cu") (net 15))
 (segment (start 61.139456 143.6624) (end 73.0076 143.6624) (width 0.15) (layer "F.Cu") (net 15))
 (segment (start 73.0076 143.6624) (end 74.63 142.04) (width 0.3) (layer "F.Cu") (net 15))
 (segment (start 54.617488 162.095312) (end 51.9684 164.7444) (width 0.3) (layer "F.Cu") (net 15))
 (segment (start 58.501856 146.3) (end 61.139456 143.6624) (width 0.15) (layer "F.Cu") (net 15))
 (segment (start 51.9814 169.866968) (end 51.9814 170.5) (width 0.3) (layer "F.Cu") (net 15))
 (segment (start 51.2064 166.4625) (end 51.2064 169.091968) (width 0.3) (layer "F.Cu") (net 15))
 (segment (start 64.545313 152.625) (end 64.553125 152.617188) (width 0.3) (layer "F.Cu") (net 15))
 (segment (start 64.545313 162.095312) (end 64.545313 152.625) (width 0.3) (layer "F.Cu") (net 15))
 (segment (start 51.2064 165.5064) (end 51.2064 166.4625) (width 0.3) (layer "F.Cu") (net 15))
 (segment (start 54.0761 170.5) (end 54.3052 170.2709) (width 0.3) (layer "F.Cu") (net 15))
 (segment (start 51.9814 170.5) (end 54.0761 170.5) (width 0.3) (layer "F.Cu") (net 15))
 (segment (start 64.553125 152.617188) (end 64.553125 152.116875) (width 0.3) (layer "F.Cu") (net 15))
 (segment (start 50.4184 166.3005) (end 50.2564 166.4625) (width 0.3) (layer "F.Cu") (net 9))
 (segment (start 64.6 168.725) (end 68.275 168.725) (width 0.3) (layer "F.Cu") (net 9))
 (segment (start 59.4086 145.925) (end 50.4184 154.9152) (width 0.3) (layer "F.Cu") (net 9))
 (segment (start 50.4184 164.7444) (end 50.4184 166.3005) (width 0.3) (layer "F.Cu") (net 9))
 (segment (start 50.4184 154.9152) (end 50.4184 164.7444) (width 0.3) (layer "F.Cu") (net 9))
 (segment (start 64.6 147.912) (end 64.6176 147.9296) (width 0.3) (layer "F.Cu") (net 9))
 (segment (start 64.6 145.925) (end 59.4086 145.925) (width 0.3) (layer "F.Cu") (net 9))
 (segment (start 64.6 145.925) (end 64.6 147.912) (width 0.3) (layer "F.Cu") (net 9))
 (segment (start 64.7192 166.7764) (end 64.7192 168.6058) (width 0.3) (layer "F.Cu") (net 9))
 (segment (start 68.275 168.725) (end 72.09 172.54) (width 0.3) (layer "F.Cu") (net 9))
 (segment (start 64.7192 168.6058) (end 64.6 168.725) (width 0.3) (layer "F.Cu") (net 9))
 (via (at 64.6176 147.9296) (size 0.6) (drill 0.3) (layers "F.Cu" "B.Cu") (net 9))
 (via (at 64.7192 166.7764) (size 0.6) (drill 0.3) (layers "F.Cu" "B.Cu") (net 9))
 (segment (start 64.6176 166.6748) (end 64.7192 166.7764) (width 0.3) (layer "B.Cu") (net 9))
 (segment (start 64.6176 147.9296) (end 64.6176 166.6748) (width 0.3) (layer "B.Cu") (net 9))
 (segment (start 50.2564 168.7375) (end 50.2564 171.0264) (width 0.3) (layer "F.Cu") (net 1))
 (segment (start 50.2564 171.0264) (end 51.77 172.54) (width 0.3) (layer "F.Cu") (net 1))
 (segment (start 56.85 142.04) (end 50.59 148.3) (width 0.15) (layer "B.Cu") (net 22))
 (segment (start 50.59 148.3) (end 50.147 148.3) (width 0.15) (layer "B.Cu") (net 22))
 (segment (start 54.31 143.10066) (end 52.11066 145.3) (width 0.15) (layer "B.Cu") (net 23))
 (segment (start 52.11066 145.3) (end 50.147 145.3) (width 0.15) (layer "B.Cu") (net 23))
 (segment (start 54.31 142.04) (end 54.31 143.10066) (width 0.15) (layer "B.Cu") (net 23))
 (segment (start 50.147 144.3) (end 49.496 144.951) (width 0.15) (layer "F.Cu") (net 8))
 (segment (start 50.735695 173.516) (end 68.574 173.516) (width 0.15) (layer "F.Cu") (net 8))
 (segment (start 49.496 172.276305) (end 50.735695 173.516) (width 0.15) (layer "F.Cu") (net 8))
 (segment (start 49.496 144.951) (end 49.496 172.276305) (width 0.15) (layer "F.Cu") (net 8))
 (segment (start 68.574 173.516) (end 69.55 172.54) (width 0.15) (layer "F.Cu") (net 8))
 (segment (start 49.496 146.649) (end 49.496 142.362) (width 0.15) (layer "B.Cu") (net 21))
 (segment (start 49.496 142.362) (end 50.794 141.064) (width 0.15) (layer "B.Cu") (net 21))
 (segment (start 50.794 141.064) (end 58.414 141.064) (width 0.15) (layer "B.Cu") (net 21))
 (segment (start 58.414 141.064) (end 59.39 142.04) (width 0.15) (layer "B.Cu") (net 21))
 (segment (start 50.147 147.3) (end 49.496 146.649) (width 0.15) (layer "B.Cu") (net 21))
 (segment (start 52.9136 168.7375) (end 54.3052 167.3459) (width 0.3) (layer "F.Cu") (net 27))
 (segment (start 52.1564 168.7375) (end 52.9136 168.7375) (width 0.3) (layer "F.Cu") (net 27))
 (segment (start 50.147 160.757) (end 61.93 172.54) (width 0.15) (layer "B.Cu") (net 5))
 (segment (start 50.147 149.3) (end 50.147 160.757) (width 0.15) (layer "B.Cu") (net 5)))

